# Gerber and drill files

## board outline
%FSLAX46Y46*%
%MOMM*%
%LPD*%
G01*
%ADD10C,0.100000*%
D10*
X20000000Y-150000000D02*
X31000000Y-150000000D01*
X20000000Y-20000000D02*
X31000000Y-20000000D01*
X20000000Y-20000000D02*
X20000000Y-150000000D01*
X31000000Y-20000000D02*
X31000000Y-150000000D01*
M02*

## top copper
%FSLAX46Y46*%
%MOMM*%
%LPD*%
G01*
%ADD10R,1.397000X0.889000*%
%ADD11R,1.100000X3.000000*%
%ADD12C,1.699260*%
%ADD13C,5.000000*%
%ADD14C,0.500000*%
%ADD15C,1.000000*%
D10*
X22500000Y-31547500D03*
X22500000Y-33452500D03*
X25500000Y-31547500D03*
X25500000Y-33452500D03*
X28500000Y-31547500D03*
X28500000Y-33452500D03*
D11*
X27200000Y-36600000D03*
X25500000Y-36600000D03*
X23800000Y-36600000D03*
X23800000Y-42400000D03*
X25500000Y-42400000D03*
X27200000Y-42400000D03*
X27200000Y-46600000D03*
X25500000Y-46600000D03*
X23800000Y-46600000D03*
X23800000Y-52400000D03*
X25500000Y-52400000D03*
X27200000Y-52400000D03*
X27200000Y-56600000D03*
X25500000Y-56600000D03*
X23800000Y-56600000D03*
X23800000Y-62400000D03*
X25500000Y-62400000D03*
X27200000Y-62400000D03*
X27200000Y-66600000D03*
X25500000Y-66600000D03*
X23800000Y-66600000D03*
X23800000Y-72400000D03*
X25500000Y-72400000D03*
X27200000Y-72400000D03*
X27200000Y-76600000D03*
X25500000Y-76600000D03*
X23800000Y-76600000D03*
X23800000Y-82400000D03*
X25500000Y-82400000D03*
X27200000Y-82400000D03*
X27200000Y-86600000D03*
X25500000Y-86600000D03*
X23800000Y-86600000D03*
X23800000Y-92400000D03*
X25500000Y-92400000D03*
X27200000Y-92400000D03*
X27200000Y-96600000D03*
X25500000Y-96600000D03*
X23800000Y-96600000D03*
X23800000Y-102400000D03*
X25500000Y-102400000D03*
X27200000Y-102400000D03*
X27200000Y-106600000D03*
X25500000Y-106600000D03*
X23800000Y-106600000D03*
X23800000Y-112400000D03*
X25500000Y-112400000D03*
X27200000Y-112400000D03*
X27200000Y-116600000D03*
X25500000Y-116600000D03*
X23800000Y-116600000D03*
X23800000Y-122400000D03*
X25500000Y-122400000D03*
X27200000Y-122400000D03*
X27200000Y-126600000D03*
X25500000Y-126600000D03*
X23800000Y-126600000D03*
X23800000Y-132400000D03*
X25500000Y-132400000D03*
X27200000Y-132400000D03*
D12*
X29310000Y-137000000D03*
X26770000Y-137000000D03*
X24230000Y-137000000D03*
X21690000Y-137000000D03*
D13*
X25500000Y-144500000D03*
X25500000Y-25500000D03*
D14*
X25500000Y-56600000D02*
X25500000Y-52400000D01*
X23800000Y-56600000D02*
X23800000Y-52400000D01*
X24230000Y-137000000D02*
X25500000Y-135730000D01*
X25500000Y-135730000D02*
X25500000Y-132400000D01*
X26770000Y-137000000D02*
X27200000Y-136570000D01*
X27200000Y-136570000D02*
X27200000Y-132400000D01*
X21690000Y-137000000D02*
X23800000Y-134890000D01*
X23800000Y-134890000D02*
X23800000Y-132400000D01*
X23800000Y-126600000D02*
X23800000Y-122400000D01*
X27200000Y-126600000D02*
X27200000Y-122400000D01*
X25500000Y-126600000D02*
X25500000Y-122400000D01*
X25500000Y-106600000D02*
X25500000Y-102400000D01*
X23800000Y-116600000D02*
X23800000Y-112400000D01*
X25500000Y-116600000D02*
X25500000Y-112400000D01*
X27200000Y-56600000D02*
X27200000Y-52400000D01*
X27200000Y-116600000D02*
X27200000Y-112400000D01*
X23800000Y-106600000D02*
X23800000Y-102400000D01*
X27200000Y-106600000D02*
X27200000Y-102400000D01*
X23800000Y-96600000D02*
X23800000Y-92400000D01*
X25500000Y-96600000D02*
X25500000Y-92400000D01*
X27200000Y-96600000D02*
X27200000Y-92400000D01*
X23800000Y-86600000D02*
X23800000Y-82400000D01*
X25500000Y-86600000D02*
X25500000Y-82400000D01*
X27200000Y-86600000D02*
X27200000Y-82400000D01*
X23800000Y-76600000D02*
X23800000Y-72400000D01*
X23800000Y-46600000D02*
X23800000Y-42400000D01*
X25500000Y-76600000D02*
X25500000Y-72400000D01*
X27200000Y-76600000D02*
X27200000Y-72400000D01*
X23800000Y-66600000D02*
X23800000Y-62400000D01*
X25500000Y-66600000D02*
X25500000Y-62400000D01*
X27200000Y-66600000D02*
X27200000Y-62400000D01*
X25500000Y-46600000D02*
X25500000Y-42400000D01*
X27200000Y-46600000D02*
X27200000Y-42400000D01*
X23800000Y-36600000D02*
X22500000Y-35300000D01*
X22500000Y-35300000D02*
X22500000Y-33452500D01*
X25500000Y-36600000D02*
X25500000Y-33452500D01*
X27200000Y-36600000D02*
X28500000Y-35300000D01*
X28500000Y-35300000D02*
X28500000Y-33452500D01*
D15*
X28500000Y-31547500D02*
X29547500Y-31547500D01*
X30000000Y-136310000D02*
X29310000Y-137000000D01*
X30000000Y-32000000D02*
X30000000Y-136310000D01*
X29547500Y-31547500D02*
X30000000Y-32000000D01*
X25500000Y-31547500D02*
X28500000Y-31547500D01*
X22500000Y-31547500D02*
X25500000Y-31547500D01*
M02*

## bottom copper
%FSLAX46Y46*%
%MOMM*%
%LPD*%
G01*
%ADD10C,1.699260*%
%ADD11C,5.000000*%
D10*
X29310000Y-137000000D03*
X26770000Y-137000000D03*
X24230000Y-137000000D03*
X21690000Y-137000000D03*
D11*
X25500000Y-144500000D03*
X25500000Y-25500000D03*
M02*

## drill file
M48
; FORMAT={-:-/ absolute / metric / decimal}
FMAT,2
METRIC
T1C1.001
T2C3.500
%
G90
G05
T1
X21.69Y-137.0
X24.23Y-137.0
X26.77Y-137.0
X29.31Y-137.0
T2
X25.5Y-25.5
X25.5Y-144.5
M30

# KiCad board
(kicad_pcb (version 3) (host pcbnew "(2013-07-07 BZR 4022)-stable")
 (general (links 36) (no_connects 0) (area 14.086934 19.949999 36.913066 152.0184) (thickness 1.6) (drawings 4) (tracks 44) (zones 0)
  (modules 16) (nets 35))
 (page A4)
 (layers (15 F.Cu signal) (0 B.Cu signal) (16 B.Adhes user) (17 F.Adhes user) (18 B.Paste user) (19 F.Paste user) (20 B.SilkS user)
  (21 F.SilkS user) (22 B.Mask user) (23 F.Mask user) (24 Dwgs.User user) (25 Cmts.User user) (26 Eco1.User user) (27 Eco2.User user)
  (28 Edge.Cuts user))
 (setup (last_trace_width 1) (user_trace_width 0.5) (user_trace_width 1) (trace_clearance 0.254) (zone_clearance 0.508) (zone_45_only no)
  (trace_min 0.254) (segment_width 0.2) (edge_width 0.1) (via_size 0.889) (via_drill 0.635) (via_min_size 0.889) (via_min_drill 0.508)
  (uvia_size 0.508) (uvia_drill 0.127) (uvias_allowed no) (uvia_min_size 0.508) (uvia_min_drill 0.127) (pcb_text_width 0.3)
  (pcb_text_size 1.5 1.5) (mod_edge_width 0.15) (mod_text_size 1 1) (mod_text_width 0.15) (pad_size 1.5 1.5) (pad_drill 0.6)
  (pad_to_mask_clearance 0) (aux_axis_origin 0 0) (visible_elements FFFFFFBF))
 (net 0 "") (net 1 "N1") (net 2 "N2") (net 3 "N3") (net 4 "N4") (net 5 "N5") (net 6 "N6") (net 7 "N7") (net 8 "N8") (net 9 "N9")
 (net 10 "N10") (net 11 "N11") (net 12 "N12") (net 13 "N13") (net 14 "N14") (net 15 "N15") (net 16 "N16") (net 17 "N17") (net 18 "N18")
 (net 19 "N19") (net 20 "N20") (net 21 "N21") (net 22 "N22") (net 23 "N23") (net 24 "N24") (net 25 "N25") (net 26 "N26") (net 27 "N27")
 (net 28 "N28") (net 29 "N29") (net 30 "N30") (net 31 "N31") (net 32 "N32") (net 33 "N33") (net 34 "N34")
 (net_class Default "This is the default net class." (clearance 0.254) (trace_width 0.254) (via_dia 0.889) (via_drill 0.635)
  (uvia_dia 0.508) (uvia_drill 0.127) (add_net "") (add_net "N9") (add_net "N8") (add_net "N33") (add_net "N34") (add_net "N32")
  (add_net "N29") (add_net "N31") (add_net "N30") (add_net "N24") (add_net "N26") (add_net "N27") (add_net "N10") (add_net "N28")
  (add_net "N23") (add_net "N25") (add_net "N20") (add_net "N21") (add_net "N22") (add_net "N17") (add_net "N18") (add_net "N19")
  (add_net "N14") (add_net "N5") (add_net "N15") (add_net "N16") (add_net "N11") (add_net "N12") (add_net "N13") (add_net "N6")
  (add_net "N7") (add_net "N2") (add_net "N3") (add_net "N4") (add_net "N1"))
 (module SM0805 (layer F.Cu) (at 22.5 32.5 270)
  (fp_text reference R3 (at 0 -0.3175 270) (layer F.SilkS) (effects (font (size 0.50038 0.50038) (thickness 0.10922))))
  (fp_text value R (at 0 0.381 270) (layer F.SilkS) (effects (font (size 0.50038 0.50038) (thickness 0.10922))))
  (pad 1 smd rect (at -0.9525 0 270) (size 0.889 1.397) (layers F.Cu F.Paste F.Mask) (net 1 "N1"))
  (pad 2 smd rect (at 0.9525 0 270) (size 0.889 1.397) (layers F.Cu F.Paste F.Mask) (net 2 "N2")))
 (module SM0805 (layer F.Cu) (at 25.5 32.5 270)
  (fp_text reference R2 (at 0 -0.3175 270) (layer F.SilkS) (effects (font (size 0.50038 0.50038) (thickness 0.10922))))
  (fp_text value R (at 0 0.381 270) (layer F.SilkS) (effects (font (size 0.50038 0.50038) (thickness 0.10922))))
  (pad 1 smd rect (at -0.9525 0 270) (size 0.889 1.397) (layers F.Cu F.Paste F.Mask) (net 1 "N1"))
  (pad 2 smd rect (at 0.9525 0 270) (size 0.889 1.397) (layers F.Cu F.Paste F.Mask) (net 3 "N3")))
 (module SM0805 (layer F.Cu) (at 28.5 32.5 270)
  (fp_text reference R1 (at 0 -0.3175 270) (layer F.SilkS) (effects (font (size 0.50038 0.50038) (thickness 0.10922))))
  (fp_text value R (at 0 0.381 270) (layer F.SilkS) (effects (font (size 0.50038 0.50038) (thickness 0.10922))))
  (pad 1 smd rect (at -0.9525 0 270) (size 0.889 1.397) (layers F.Cu F.Paste F.Mask) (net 1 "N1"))
  (pad 2 smd rect (at 0.9525 0 270) (size 0.889 1.397) (layers F.Cu F.Paste F.Mask) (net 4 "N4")))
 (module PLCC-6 (layer F.Cu) (at 25.5 39.5 180)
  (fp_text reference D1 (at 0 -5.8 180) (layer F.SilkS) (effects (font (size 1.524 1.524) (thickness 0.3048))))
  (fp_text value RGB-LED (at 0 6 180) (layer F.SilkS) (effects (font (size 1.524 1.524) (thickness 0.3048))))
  (pad 1 smd rect (at -1.7 2.9 180) (size 1.1 3) (layers F.Cu F.Paste F.Mask) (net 4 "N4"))
  (pad 2 smd rect (at 0 2.9 180) (size 1.1 3) (layers F.Cu F.Paste F.Mask) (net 3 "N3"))
  (pad 3 smd rect (at 1.7 2.9 180) (size 1.1 3) (layers F.Cu F.Paste F.Mask) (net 2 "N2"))
  (pad 4 smd rect (at 1.7 -2.9 180) (size 1.1 3) (layers F.Cu F.Paste F.Mask) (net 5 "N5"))
  (pad 5 smd rect (at 0 -2.9 180) (size 1.1 3) (layers F.Cu F.Paste F.Mask) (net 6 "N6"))
  (pad 6 smd rect (at -1.7 -2.9 180) (size 1.1 3) (layers F.Cu F.Paste F.Mask) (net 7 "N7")))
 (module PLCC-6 (layer F.Cu) (at 25.5 49.5 180)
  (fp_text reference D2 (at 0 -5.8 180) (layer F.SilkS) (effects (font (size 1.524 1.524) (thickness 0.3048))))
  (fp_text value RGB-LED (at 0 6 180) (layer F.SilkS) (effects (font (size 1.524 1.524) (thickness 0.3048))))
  (pad 1 smd rect (at -1.7 2.9 180) (size 1.1 3) (layers F.Cu F.Paste F.Mask) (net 7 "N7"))
  (pad 2 smd rect (at 0 2.9 180) (size 1.1 3) (layers F.Cu F.Paste F.Mask) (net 6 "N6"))
  (pad 3 smd rect (at 1.7 2.9 180) (size 1.1 3) (layers F.Cu F.Paste F.Mask) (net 5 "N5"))
  (pad 4 smd rect (at 1.7 -2.9 180) (size 1.1 3) (layers F.Cu F.Paste F.Mask) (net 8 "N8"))
  (pad 5 smd rect (at 0 -2.9 180) (size 1.1 3) (layers F.Cu F.Paste F.Mask) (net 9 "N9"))
  (pad 6 smd rect (at -1.7 -2.9 180) (size 1.1 3) (layers F.Cu F.Paste F.Mask) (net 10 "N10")))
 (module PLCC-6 (layer F.Cu) (at 25.5 59.5 180)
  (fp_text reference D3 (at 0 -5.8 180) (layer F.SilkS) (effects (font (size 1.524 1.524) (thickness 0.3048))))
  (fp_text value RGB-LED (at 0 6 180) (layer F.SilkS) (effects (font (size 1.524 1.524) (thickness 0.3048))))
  (pad 1 smd rect (at -1.7 2.9 180) (size 1.1 3) (layers F.Cu F.Paste F.Mask) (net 10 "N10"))
  (pad 2 smd rect (at 0 2.9 180) (size 1.1 3) (layers F.Cu F.Paste F.Mask) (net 9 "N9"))
  (pad 3 smd rect (at 1.7 2.9 180) (size 1.1 3) (layers F.Cu F.Paste F.Mask) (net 8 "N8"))
  (pad 4 smd rect (at 1.7 -2.9 180) (size 1.1 3) (layers F.Cu F.Paste F.Mask) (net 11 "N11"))
  (pad 5 smd rect (at 0 -2.9 180) (size 1.1 3) (layers F.Cu F.Paste F.Mask) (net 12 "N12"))
  (pad 6 smd rect (at -1.7 -2.9 180) (size 1.1 3) (layers F.Cu F.Paste F.Mask) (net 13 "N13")))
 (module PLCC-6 (layer F.Cu) (at 25.5 69.5 180)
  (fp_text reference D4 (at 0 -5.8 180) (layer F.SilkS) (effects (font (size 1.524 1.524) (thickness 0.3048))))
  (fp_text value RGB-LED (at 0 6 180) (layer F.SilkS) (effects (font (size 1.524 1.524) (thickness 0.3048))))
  (pad 1 smd rect (at -1.7 2.9 180) (size 1.1 3) (layers F.Cu F.Paste F.Mask) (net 13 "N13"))
  (pad 2 smd rect (at 0 2.9 180) (size 1.1 3) (layers F.Cu F.Paste F.Mask) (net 12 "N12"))
  (pad 3 smd rect (at 1.7 2.9 180) (size 1.1 3) (layers F.Cu F.Paste F.Mask) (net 11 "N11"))
  (pad 4 smd rect (at 1.7 -2.9 180) (size 1.1 3) (layers F.Cu F.Paste F.Mask) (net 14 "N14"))
  (pad 5 smd rect (at 0 -2.9 180) (size 1.1 3) (layers F.Cu F.Paste F.Mask) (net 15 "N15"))
  (pad 6 smd rect (at -1.7 -2.9 180) (size 1.1 3) (layers F.Cu F.Paste F.Mask) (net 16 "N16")))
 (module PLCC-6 (layer F.Cu) (at 25.5 79.5 180)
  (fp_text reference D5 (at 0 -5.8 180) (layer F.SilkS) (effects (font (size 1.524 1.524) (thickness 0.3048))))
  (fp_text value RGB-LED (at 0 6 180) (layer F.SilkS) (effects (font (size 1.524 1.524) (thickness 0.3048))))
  (pad 1 smd rect (at -1.7 2.9 180) (size 1.1 3) (layers F.Cu F.Paste F.Mask) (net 16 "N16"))
  (pad 2 smd rect (at 0 2.9 180) (size 1.1 3) (layers F.Cu F.Paste F.Mask) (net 15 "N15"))
  (pad 3 smd rect (at 1.7 2.9 180) (size 1.1 3) (layers F.Cu F.Paste F.Mask) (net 14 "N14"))
  (pad 4 smd rect (at 1.7 -2.9 180) (size 1.1 3) (layers F.Cu F.Paste F.Mask) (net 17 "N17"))
  (pad 5 smd rect (at 0 -2.9 180) (size 1.1 3) (layers F.Cu F.Paste F.Mask) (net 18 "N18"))
  (pad 6 smd rect (at -1.7 -2.9 180) (size 1.1 3) (layers F.Cu F.Paste F.Mask) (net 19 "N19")))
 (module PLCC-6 (layer F.Cu) (at 25.5 89.5 180)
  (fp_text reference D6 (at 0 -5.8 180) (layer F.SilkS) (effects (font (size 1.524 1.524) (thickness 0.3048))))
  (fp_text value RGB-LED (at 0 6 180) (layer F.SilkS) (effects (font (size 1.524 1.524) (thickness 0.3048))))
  (pad 1 smd rect (at -1.7 2.9 180) (size 1.1 3) (layers F.Cu F.Paste F.Mask) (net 19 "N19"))
  (pad 2 smd rect (at 0 2.9 180) (size 1.1 3) (layers F.Cu F.Paste F.Mask) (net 18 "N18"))
  (pad 3 smd rect (at 1.7 2.9 180) (size 1.1 3) (layers F.Cu F.Paste F.Mask) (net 17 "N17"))
  (pad 4 smd rect (at 1.7 -2.9 180) (size 1.1 3) (layers F.Cu F.Paste F.Mask) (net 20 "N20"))
  (pad 5 smd rect (at 0 -2.9 180) (size 1.1 3) (layers F.Cu F.Paste F.Mask) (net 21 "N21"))
  (pad 6 smd rect (at -1.7 -2.9 180) (size 1.1 3) (layers F.Cu F.Paste F.Mask) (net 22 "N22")))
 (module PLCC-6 (layer F.Cu) (at 25.5 99.5 180)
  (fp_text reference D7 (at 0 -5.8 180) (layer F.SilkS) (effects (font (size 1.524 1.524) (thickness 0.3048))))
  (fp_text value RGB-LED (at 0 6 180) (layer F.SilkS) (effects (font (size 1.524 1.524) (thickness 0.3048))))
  (pad 1 smd rect (at -1.7 2.9 180) (size 1.1 3) (layers F.Cu F.Paste F.Mask) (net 22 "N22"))
  (pad 2 smd rect (at 0 2.9 180) (size 1.1 3) (layers F.Cu F.Paste F.Mask) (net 21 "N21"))
  (pad 3 smd rect (at 1.7 2.9 180) (size 1.1 3) (layers F.Cu F.Paste F.Mask) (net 20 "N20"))
  (pad 4 smd rect (at 1.7 -2.9 180) (size 1.1 3) (layers F.Cu F.Paste F.Mask) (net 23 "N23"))
  (pad 5 smd rect (at 0 -2.9 180) (size 1.1 3) (layers F.Cu F.Paste F.Mask) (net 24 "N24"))
  (pad 6 smd rect (at -1.7 -2.9 180) (size 1.1 3) (layers F.Cu F.Paste F.Mask) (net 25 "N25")))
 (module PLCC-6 (layer F.Cu) (at 25.5 109.5 180)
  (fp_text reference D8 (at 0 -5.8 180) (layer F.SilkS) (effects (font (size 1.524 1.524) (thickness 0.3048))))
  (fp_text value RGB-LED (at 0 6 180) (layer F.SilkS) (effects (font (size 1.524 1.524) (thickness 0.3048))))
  (pad 1 smd rect (at -1.7 2.9 180) (size 1.1 3) (layers F.Cu F.Paste F.Mask) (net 25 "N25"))
  (pad 2 smd rect (at 0 2.9 180) (size 1.1 3) (layers F.Cu F.Paste F.Mask) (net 24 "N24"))
  (pad 3 smd rect (at 1.7 2.9 180) (size 1.1 3) (layers F.Cu F.Paste F.Mask) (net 23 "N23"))
  (pad 4 smd rect (at 1.7 -2.9 180) (size 1.1 3) (layers F.Cu F.Paste F.Mask) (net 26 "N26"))
  (pad 5 smd rect (at 0 -2.9 180) (size 1.1 3) (layers F.Cu F.Paste F.Mask) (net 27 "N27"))
  (pad 6 smd rect (at -1.7 -2.9 180) (size 1.1 3) (layers F.Cu F.Paste F.Mask) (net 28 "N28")))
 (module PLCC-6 (layer F.Cu) (at 25.5 119.5 180)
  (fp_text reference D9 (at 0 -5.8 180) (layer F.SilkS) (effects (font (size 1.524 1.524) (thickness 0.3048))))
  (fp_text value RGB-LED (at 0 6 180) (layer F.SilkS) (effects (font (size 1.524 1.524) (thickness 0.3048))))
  (pad 1 smd rect (at -1.7 2.9 180) (size 1.1 3) (layers F.Cu F.Paste F.Mask) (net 28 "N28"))
  (pad 2 smd rect (at 0 2.9 180) (size 1.1 3) (layers F.Cu F.Paste F.Mask) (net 27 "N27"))
  (pad 3 smd rect (at 1.7 2.9 180) (size 1.1 3) (layers F.Cu F.Paste F.Mask) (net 26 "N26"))
  (pad 4 smd rect (at 1.7 -2.9 180) (size 1.1 3) (layers F.Cu F.Paste F.Mask) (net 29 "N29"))
  (pad 5 smd rect (at 0 -2.9 180) (size 1.1 3) (layers F.Cu F.Paste F.Mask) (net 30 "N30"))
  (pad 6 smd rect (at -1.7 -2.9 180) (size 1.1 3) (layers F.Cu F.Paste F.Mask) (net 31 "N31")))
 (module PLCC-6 (layer F.Cu) (at 25.5 129.5 180)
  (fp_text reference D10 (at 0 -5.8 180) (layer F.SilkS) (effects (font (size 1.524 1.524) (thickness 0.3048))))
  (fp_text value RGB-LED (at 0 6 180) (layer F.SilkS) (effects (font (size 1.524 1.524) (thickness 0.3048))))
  (pad 1 smd rect (at -1.7 2.9 180) (size 1.1 3) (layers F.Cu F.Paste F.Mask) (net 31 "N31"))
  (pad 2 smd rect (at 0 2.9 180) (size 1.1 3) (layers F.Cu F.Paste F.Mask) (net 30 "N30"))
  (pad 3 smd rect (at 1.7 2.9 180) (size 1.1 3) (layers F.Cu F.Paste F.Mask) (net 29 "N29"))
  (pad 4 smd rect (at 1.7 -2.9 180) (size 1.1 3) (layers F.Cu F.Paste F.Mask) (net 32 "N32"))
  (pad 5 smd rect (at 0 -2.9 180) (size 1.1 3) (layers F.Cu F.Paste F.Mask) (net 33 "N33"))
  (pad 6 smd rect (at -1.7 -2.9 180) (size 1.1 3) (layers F.Cu F.Paste F.Mask) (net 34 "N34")))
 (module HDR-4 (layer F.Cu) (at 25.5 137 180)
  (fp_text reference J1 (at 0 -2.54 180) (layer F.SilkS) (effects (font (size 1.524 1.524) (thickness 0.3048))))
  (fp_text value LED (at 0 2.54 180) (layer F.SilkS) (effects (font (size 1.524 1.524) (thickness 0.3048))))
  (pad 1 thru_hole circle (at -3.81 0 180) (size 1.69926 1.69926) (drill 1.00076) (layers *.Cu *.Mask F.SilkS) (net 1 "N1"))
  (pad 2 thru_hole circle (at -1.27 0 180) (size 1.69926 1.69926) (drill 1.00076) (layers *.Cu *.Mask F.SilkS) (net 34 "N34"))
  (pad 3 thru_hole circle (at 1.27 0 180) (size 1.69926 1.69926) (drill 1.00076) (layers *.Cu *.Mask F.SilkS) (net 33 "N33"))
  (pad 4 thru_hole circle (at 3.81 0 180) (size 1.69926 1.69926) (drill 1.00076) (layers *.Cu *.Mask F.SilkS) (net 32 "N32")))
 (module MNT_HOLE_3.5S (layer F.Cu) (at 25.5 144.5 180)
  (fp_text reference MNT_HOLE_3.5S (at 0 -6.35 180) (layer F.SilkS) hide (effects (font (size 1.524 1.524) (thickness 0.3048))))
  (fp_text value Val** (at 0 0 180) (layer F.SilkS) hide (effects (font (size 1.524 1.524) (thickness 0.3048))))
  (pad "" thru_hole circle (at 0 0 180) (size 5 5) (drill 3.5) (layers *.Cu *.Mask F.SilkS)))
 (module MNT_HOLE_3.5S (layer F.Cu) (at 25.5 25.5 180)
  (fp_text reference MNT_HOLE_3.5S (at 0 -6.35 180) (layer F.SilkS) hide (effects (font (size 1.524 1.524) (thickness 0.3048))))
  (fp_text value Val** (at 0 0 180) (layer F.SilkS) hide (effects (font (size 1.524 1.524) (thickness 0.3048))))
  (pad "" thru_hole circle (at 0 0 180) (size 5 5) (drill 3.5) (layers *.Cu *.Mask F.SilkS)))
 (gr_line (start 20 150) (end 31 150) (angle 90) (layer Edge.Cuts) (width 0.1))
 (gr_line (start 20 20) (end 31 20) (angle 90) (layer Edge.Cuts) (width 0.1))
 (gr_line (start 20 20) (end 20 150) (angle 90) (layer Edge.Cuts) (width 0.1))
 (gr_line (start 31 20) (end 31 150) (angle 90) (layer Edge.Cuts) (width 0.1))
 (segment (start 25.5 56.6) (end 25.5 52.4) (width 0.5) (layer F.Cu) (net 9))
 (segment (start 23.8 56.6) (end 23.8 52.4) (width 0.5) (layer F.Cu) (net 8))
 (segment (start 24.23 137) (end 25.5 135.73) (width 0.5) (layer F.Cu) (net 33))
 (segment (start 25.5 135.73) (end 25.5 132.4) (width 0.5) (layer F.Cu) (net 33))
 (segment (start 26.77 137) (end 27.2 136.57) (width 0.5) (layer F.Cu) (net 34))
 (segment (start 27.2 136.57) (end 27.2 132.4) (width 0.5) (layer F.Cu) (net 34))
 (segment (start 21.69 137) (end 23.8 134.89) (width 0.5) (layer F.Cu) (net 32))
 (segment (start 23.8 134.89) (end 23.8 132.4) (width 0.5) (layer F.Cu) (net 32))
 (segment (start 23.8 126.6) (end 23.8 122.4) (width 0.5) (layer F.Cu) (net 29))
 (segment (start 27.2 126.6) (end 27.2 122.4) (width 0.5) (layer F.Cu) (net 31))
 (segment (start 25.5 126.6) (end 25.5 122.4) (width 0.5) (layer F.Cu) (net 30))
 (segment (start 25.5 106.6) (end 25.5 102.4) (width 0.5) (layer F.Cu) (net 24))
 (segment (start 23.8 116.6) (end 23.8 112.4) (width 0.5) (layer F.Cu) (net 26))
 (segment (start 25.5 116.6) (end 25.5 112.4) (width 0.5) (layer F.Cu) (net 27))
 (segment (start 27.2 56.6) (end 27.2 52.4) (width 0.5) (layer F.Cu) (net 10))
 (segment (start 27.2 116.6) (end 27.2 112.4) (width 0.5) (layer F.Cu) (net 28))
 (segment (start 23.8 106.6) (end 23.8 102.4) (width 0.5) (layer F.Cu) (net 23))
 (segment (start 27.2 106.6) (end 27.2 102.4) (width 0.5) (layer F.Cu) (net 25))
 (segment (start 23.8 96.6) (end 23.8 92.4) (width 0.5) (layer F.Cu) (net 20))
 (segment (start 25.5 96.6) (end 25.5 92.4) (width 0.5) (layer F.Cu) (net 21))
 (segment (start 27.2 96.6) (end 27.2 92.4) (width 0.5) (layer F.Cu) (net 22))
 (segment (start 23.8 86.6) (end 23.8 82.4) (width 0.5) (layer F.Cu) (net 17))
 (segment (start 25.5 86.6) (end 25.5 82.4) (width 0.5) (layer F.Cu) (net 18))
 (segment (start 27.2 86.6) (end 27.2 82.4) (width 0.5) (layer F.Cu) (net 19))
 (segment (start 23.8 76.6) (end 23.8 72.4) (width 0.5) (layer F.Cu) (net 14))
 (segment (start 23.8 46.6) (end 23.8 42.4) (width 0.5) (layer F.Cu) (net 5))
 (segment (start 25.5 76.6) (end 25.5 72.4) (width 0.5) (layer F.Cu) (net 15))
 (segment (start 27.2 76.6) (end 27.2 72.4) (width 0.5) (layer F.Cu) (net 16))
 (segment (start 23.8 66.6) (end 23.8 62.4) (width 0.5) (layer F.Cu) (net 11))
 (segment (start 25.5 66.6) (end 25.5 62.4) (width 0.5) (layer F.Cu) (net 12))
 (segment (start 27.2 66.6) (end 27.2 62.4) (width 0.5) (layer F.Cu) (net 13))
 (segment (start 25.5 46.6) (end 25.5 42.4) (width 0.5) (layer F.Cu) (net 6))
 (segment (start 27.2 46.6) (end 27.2 42.4) (width 0.5) (layer F.Cu) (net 7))
 (segment (start 23.8 36.6) (end 22.5 35.3) (width 0.5) (layer F.Cu) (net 2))
 (segment (start 22.5 35.3) (end 22.5 33.4525) (width 0.5) (layer F.Cu) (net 2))
 (segment (start 25.5 36.6) (end 25.5 33.4525) (width 0.5) (layer F.Cu) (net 3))
 (segment (start 27.2 36.6) (end 28.5 35.3) (width 0.5) (layer F.Cu) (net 4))
 (segment (start 28.5 35.3) (end 28.5 33.4525) (width 0.5) (layer F.Cu) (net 4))
 (segment (start 28.5 31.5475) (end 29.5475 31.5475) (width 1) (layer F.Cu) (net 1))
 (segment (start 30 136.31) (end 29.31 137) (width 1) (layer F.Cu) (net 1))
 (segment (start 30 32) (end 30 136.31) (width 1) (layer F.Cu) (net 1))
 (segment (start 29.5475 31.5475) (end 30 32) (width 1) (layer F.Cu) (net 1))
 (segment (start 25.5 31.5475) (end 28.5 31.5475) (width 1) (layer F.Cu) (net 1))
 (segment (start 22.5 31.5475) (end 25.5 31.5475) (width 1) (layer F.Cu) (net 1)))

